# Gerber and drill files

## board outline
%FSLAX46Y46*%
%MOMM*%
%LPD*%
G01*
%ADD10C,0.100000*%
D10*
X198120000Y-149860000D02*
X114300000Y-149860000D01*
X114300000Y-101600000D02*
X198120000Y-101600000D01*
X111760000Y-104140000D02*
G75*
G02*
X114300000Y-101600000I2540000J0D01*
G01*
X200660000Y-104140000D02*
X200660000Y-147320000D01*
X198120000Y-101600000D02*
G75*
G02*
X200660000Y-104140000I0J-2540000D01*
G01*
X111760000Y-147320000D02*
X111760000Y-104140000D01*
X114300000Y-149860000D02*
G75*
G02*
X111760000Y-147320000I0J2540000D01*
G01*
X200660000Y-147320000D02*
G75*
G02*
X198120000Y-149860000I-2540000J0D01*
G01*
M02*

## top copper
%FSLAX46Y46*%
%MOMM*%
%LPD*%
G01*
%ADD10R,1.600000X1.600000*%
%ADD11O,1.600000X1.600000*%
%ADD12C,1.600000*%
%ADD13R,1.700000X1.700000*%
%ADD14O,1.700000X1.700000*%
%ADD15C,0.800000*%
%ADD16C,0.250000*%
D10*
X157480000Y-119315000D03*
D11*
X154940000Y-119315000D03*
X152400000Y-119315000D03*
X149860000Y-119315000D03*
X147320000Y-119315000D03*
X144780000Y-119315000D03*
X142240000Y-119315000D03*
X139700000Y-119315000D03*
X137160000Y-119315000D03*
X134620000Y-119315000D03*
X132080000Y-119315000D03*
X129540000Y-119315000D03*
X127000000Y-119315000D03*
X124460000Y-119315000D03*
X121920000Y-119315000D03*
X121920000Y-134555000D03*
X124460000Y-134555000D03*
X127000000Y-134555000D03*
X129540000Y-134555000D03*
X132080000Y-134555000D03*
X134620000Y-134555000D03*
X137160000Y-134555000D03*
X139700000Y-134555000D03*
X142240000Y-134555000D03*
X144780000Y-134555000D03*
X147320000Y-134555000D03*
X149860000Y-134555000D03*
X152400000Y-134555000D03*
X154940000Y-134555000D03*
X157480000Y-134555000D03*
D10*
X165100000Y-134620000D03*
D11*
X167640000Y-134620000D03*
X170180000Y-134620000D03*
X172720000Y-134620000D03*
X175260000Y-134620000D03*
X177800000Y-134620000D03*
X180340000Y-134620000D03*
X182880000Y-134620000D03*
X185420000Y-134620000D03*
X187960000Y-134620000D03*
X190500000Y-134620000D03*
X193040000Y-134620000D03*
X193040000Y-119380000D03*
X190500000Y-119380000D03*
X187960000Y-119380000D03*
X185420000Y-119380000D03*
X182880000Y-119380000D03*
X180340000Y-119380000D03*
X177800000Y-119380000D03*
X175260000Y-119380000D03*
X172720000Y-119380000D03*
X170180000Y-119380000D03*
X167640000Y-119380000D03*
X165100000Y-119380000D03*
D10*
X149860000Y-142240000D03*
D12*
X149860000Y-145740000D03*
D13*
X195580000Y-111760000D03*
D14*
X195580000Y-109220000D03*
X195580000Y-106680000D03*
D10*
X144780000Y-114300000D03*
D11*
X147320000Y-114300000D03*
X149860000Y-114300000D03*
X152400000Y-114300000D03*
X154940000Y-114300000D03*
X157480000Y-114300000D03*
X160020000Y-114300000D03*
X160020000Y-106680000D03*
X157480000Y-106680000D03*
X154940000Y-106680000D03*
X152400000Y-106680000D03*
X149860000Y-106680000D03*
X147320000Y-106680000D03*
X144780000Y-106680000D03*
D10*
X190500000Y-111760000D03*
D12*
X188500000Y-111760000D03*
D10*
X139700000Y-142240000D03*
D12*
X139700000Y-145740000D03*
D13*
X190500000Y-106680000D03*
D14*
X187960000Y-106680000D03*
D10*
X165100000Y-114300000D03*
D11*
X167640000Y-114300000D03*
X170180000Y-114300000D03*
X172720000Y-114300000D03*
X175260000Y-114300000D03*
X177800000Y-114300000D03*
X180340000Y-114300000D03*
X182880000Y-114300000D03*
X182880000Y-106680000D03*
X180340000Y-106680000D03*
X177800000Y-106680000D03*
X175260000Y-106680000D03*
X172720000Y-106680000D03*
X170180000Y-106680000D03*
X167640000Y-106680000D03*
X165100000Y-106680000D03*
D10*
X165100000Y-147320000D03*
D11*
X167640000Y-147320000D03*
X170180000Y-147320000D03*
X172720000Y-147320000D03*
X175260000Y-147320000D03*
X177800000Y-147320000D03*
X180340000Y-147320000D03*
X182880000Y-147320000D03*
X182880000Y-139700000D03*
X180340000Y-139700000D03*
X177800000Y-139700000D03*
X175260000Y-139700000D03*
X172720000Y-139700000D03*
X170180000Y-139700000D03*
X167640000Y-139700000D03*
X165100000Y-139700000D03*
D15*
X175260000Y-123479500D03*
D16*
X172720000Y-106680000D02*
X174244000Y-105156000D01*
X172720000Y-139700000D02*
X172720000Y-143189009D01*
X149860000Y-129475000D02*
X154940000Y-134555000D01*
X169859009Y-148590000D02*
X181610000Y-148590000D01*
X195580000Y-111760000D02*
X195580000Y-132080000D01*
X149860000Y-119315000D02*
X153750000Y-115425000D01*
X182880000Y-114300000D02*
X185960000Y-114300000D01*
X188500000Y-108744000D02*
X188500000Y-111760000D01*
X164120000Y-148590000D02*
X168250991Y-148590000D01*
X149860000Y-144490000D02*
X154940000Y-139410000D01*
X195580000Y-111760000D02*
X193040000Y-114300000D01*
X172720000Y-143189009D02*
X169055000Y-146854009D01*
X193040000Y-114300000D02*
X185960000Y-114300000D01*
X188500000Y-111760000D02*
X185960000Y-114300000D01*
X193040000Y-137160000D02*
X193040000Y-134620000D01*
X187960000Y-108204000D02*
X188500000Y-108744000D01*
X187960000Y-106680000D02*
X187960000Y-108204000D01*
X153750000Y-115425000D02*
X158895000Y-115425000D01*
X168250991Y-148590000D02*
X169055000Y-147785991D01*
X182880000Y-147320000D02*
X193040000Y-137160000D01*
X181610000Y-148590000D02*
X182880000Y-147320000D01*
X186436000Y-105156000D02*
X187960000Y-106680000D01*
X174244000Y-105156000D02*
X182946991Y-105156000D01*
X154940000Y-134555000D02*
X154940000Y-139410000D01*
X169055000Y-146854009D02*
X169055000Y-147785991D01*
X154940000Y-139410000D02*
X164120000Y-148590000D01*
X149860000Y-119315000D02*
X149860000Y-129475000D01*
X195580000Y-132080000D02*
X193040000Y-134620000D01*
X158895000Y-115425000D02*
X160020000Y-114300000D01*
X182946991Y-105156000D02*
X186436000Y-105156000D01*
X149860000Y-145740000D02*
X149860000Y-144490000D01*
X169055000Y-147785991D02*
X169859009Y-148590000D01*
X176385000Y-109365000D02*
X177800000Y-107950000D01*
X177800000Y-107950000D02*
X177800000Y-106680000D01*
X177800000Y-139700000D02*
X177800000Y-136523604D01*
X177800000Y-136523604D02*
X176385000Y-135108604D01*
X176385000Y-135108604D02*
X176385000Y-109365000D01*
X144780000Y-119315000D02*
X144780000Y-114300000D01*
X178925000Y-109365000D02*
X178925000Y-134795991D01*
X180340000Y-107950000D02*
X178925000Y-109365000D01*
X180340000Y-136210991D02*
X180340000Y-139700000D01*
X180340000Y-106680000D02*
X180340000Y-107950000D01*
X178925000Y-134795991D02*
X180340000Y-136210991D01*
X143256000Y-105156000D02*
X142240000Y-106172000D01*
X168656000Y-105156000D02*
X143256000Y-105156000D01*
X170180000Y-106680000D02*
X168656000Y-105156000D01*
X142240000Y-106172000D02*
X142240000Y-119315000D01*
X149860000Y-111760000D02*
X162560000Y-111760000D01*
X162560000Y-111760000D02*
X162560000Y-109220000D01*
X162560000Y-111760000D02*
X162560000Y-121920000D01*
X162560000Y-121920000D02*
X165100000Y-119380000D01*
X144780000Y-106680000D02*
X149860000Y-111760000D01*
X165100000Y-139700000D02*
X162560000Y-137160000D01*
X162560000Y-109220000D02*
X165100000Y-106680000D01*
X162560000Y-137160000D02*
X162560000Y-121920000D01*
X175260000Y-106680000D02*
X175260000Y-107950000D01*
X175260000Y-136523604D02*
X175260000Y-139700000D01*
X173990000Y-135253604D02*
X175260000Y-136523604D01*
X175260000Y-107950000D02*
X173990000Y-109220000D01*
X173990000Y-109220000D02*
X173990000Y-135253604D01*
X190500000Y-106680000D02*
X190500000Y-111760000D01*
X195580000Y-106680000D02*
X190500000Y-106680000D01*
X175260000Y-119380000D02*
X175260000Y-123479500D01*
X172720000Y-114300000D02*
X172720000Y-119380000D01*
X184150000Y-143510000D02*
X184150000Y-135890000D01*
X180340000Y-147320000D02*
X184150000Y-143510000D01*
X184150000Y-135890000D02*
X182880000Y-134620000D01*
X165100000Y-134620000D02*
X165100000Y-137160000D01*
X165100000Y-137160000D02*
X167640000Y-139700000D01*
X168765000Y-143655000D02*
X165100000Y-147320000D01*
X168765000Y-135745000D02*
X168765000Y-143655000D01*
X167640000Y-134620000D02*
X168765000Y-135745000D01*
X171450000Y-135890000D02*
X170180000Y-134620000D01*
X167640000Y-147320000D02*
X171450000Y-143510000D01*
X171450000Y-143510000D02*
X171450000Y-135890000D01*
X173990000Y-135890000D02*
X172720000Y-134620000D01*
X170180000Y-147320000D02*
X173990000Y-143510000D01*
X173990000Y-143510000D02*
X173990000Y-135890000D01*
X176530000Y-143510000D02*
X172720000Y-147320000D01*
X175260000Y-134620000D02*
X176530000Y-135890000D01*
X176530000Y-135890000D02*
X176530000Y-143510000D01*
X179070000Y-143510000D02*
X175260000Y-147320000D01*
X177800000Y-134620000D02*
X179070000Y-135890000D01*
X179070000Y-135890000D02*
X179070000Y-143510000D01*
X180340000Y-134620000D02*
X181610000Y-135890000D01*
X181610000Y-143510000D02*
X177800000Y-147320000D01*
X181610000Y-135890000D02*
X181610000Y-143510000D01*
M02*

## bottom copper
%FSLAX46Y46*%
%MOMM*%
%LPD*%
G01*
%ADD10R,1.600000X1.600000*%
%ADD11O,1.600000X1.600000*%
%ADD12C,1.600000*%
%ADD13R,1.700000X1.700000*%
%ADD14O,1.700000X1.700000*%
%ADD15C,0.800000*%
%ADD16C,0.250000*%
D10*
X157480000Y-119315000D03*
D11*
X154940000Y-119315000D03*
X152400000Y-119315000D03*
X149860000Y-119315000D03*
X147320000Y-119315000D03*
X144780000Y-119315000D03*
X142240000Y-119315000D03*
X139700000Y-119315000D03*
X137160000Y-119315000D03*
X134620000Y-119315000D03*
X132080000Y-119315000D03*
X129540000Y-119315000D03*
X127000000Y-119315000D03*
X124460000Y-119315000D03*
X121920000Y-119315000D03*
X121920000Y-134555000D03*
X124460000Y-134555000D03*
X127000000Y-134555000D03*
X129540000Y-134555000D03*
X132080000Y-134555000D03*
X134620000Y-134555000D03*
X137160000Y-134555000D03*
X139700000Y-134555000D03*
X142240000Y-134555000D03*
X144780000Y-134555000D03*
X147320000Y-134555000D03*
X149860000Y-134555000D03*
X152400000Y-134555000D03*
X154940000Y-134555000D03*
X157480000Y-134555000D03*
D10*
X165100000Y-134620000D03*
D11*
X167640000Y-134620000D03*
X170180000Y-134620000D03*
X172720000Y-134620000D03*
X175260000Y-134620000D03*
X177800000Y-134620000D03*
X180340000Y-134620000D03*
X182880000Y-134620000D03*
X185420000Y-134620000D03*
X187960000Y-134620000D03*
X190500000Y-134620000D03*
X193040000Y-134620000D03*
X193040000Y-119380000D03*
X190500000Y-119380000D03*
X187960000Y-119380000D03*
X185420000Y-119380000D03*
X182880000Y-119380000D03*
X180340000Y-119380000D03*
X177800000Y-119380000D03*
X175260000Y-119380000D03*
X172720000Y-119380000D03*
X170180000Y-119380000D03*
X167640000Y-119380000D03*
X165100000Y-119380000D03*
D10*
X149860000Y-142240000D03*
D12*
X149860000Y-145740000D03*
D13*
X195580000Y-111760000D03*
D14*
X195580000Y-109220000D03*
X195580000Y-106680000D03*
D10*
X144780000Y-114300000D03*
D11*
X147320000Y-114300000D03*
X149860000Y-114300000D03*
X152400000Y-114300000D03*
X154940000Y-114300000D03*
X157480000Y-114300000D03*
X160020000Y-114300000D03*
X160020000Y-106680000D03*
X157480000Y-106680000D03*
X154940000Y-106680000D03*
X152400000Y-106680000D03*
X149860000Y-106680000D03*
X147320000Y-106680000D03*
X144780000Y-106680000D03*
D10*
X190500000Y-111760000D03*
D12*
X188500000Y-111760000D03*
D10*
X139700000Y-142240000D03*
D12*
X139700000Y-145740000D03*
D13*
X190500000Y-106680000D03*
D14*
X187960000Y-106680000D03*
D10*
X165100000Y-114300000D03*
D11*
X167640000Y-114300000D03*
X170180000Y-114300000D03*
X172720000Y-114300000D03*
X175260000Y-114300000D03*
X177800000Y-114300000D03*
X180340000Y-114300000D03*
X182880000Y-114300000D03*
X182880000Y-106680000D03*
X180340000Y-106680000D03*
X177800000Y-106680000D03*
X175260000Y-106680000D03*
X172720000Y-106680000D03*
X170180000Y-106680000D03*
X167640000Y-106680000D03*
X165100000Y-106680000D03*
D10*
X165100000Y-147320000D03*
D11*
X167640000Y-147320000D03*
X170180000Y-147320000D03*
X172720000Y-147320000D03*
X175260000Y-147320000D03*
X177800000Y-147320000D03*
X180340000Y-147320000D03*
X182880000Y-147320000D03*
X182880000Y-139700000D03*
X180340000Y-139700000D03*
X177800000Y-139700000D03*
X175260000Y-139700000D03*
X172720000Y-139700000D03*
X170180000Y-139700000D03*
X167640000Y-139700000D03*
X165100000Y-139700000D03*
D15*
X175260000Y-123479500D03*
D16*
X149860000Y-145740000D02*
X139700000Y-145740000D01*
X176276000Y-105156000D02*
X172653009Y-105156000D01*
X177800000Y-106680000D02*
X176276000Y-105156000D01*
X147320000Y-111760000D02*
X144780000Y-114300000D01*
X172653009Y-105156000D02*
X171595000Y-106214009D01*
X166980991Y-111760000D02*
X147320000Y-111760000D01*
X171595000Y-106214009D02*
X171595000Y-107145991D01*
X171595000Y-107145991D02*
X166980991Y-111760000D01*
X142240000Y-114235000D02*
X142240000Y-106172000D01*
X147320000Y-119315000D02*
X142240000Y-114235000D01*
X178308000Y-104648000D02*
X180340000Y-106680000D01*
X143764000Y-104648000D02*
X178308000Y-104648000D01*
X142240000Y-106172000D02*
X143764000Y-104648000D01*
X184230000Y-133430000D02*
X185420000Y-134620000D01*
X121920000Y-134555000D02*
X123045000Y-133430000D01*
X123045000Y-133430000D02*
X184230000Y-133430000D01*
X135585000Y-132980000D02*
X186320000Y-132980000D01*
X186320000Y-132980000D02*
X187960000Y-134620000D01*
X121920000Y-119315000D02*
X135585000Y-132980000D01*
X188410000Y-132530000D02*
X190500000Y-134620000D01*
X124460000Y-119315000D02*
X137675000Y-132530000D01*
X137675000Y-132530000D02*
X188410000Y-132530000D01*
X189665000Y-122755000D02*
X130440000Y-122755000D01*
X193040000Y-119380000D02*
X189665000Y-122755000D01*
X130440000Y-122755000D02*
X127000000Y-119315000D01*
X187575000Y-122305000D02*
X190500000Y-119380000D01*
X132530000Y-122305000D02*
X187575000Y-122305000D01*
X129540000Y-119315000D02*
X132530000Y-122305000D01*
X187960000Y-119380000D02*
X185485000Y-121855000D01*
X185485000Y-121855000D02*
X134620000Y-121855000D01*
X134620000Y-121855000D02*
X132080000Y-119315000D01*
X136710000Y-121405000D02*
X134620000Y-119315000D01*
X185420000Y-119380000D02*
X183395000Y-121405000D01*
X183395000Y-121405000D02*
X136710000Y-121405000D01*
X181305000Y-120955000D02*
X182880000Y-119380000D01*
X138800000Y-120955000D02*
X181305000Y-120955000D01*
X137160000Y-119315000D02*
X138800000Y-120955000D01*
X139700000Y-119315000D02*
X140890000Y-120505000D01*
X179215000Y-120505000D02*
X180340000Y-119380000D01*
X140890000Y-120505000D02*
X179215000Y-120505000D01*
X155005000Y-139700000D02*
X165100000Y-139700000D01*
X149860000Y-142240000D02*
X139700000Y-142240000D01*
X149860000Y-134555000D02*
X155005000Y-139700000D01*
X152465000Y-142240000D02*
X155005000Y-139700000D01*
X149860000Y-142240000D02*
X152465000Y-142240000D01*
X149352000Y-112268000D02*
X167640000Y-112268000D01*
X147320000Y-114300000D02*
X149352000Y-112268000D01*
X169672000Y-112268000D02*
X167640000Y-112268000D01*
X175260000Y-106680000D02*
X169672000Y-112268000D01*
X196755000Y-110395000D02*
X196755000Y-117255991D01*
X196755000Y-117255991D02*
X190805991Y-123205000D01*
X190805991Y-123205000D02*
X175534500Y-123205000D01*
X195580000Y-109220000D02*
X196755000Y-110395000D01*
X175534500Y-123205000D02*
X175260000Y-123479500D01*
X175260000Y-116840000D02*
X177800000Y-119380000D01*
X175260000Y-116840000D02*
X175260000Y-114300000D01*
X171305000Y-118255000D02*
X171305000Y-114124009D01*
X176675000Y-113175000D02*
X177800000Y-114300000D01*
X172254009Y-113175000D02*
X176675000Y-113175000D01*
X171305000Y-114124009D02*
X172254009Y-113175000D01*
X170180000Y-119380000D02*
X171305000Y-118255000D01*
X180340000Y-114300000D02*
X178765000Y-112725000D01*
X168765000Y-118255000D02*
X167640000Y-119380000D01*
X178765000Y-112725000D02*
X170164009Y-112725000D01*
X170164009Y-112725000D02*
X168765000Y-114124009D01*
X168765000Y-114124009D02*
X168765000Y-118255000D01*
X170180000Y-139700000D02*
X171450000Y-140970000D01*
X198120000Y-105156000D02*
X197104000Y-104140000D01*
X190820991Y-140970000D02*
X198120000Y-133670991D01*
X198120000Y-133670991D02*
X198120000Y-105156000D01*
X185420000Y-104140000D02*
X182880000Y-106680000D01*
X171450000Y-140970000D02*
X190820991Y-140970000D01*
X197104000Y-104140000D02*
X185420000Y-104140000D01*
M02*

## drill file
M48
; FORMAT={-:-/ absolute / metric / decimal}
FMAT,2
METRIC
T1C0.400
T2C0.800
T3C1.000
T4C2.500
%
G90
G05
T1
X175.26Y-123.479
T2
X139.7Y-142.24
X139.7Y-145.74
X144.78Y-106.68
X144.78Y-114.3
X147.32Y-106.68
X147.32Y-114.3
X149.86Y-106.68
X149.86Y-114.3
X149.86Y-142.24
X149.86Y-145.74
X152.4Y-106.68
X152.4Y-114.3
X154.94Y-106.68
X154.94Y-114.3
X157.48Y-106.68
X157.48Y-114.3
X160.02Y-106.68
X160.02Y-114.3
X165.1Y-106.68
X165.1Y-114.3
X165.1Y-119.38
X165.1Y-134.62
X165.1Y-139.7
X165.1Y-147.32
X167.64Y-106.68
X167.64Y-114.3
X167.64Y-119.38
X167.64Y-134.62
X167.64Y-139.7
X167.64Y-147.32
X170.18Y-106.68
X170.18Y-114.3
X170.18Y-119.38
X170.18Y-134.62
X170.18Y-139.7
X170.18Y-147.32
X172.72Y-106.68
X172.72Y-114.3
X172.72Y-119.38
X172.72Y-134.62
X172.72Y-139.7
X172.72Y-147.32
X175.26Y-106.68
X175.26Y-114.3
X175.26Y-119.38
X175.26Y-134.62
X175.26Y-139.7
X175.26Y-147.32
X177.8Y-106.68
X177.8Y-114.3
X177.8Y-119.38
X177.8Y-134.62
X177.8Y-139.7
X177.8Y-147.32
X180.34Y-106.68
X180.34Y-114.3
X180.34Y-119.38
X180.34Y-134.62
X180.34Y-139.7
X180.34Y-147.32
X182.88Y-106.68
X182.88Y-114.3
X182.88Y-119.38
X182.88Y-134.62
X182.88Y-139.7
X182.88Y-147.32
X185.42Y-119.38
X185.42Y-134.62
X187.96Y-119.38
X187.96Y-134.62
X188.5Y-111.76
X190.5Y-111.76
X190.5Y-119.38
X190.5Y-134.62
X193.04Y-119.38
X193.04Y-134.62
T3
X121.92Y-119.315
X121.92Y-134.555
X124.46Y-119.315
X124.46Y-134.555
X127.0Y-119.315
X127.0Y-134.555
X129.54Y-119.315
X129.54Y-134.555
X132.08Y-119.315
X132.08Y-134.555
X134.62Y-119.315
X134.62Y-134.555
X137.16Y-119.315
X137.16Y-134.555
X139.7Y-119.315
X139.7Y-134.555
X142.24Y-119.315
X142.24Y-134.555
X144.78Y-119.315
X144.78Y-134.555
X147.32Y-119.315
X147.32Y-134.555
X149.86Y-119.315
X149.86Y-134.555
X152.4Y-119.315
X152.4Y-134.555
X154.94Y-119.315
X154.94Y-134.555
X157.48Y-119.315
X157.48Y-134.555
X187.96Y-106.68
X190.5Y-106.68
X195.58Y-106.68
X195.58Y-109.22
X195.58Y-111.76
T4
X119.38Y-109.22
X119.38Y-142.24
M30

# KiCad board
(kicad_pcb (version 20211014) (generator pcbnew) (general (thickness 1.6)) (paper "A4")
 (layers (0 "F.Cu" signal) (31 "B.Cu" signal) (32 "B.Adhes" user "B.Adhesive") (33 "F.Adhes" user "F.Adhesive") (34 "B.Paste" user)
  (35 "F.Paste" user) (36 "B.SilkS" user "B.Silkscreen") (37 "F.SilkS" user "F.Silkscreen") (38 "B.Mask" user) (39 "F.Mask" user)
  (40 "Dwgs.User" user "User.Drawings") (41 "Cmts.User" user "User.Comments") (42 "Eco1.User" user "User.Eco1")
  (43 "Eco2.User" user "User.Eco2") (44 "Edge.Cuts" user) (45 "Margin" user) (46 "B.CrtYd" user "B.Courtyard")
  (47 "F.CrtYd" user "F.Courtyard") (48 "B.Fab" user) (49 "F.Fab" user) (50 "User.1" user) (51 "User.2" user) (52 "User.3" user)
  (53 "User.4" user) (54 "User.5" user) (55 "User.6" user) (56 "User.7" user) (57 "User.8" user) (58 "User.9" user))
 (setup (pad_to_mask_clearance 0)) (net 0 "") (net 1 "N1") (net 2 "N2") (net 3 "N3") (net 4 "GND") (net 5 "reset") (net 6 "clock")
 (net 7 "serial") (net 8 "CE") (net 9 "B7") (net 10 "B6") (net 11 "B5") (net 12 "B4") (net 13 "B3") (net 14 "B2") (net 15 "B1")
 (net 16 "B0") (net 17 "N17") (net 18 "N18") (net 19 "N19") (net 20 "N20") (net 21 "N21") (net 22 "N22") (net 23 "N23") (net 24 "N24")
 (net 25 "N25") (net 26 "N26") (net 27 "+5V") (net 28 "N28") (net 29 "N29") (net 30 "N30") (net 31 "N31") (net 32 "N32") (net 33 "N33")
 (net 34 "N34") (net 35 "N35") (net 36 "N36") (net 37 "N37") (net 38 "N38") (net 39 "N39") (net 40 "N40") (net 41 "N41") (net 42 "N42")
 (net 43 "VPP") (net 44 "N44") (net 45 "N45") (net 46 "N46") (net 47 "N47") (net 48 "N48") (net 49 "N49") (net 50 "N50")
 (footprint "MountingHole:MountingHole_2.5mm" (layer "F.Cu") (at 119.38 109.22)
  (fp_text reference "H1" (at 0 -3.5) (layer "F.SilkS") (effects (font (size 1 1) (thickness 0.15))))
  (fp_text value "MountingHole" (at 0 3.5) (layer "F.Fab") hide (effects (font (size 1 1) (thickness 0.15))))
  (pad "" np_thru_hole circle (at 0 0) (size 2.5 2.5) (drill 2.5) (layers *.Cu *.Mask)))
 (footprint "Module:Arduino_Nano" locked (layer "F.Cu") (at 157.48 119.315 -90)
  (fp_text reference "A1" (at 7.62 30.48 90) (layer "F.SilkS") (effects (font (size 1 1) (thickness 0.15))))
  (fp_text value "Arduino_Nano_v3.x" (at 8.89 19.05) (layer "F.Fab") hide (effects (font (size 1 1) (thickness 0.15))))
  (pad "1" thru_hole rect locked (at 0 0 270) (size 1.6 1.6) (drill 1) (layers *.Cu *.Mask) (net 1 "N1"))
  (pad "2" thru_hole oval locked (at 0 2.54 270) (size 1.6 1.6) (drill 1) (layers *.Cu *.Mask) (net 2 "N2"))
  (pad "3" thru_hole oval locked (at 0 5.08 270) (size 1.6 1.6) (drill 1) (layers *.Cu *.Mask) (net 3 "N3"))
  (pad "4" thru_hole oval locked (at 0 7.62 270) (size 1.6 1.6) (drill 1) (layers *.Cu *.Mask) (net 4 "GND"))
  (pad "5" thru_hole oval locked (at 0 10.16 270) (size 1.6 1.6) (drill 1) (layers *.Cu *.Mask) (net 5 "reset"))
  (pad "6" thru_hole oval locked (at 0 12.7 270) (size 1.6 1.6) (drill 1) (layers *.Cu *.Mask) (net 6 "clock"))
  (pad "7" thru_hole oval locked (at 0 15.24 270) (size 1.6 1.6) (drill 1) (layers *.Cu *.Mask) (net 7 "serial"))
  (pad "8" thru_hole oval locked (at 0 17.78 270) (size 1.6 1.6) (drill 1) (layers *.Cu *.Mask) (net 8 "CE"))
  (pad "9" thru_hole oval locked (at 0 20.32 270) (size 1.6 1.6) (drill 1) (layers *.Cu *.Mask) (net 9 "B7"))
  (pad "10" thru_hole oval locked (at 0 22.86 270) (size 1.6 1.6) (drill 1) (layers *.Cu *.Mask) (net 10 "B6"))
  (pad "11" thru_hole oval locked (at 0 25.4 270) (size 1.6 1.6) (drill 1) (layers *.Cu *.Mask) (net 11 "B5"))
  (pad "12" thru_hole oval locked (at 0 27.94 270) (size 1.6 1.6) (drill 1) (layers *.Cu *.Mask) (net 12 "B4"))
  (pad "13" thru_hole oval locked (at 0 30.48 270) (size 1.6 1.6) (drill 1) (layers *.Cu *.Mask) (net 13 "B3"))
  (pad "14" thru_hole oval locked (at 0 33.02 270) (size 1.6 1.6) (drill 1) (layers *.Cu *.Mask) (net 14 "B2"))
  (pad "15" thru_hole oval locked (at 0 35.56 270) (size 1.6 1.6) (drill 1) (layers *.Cu *.Mask) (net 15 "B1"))
  (pad "16" thru_hole oval locked (at 15.24 35.56 270) (size 1.6 1.6) (drill 1) (layers *.Cu *.Mask) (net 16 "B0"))
  (pad "17" thru_hole oval locked (at 15.24 33.02 270) (size 1.6 1.6) (drill 1) (layers *.Cu *.Mask) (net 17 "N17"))
  (pad "18" thru_hole oval locked (at 15.24 30.48 270) (size 1.6 1.6) (drill 1) (layers *.Cu *.Mask) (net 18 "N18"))
  (pad "19" thru_hole oval locked (at 15.24 27.94 270) (size 1.6 1.6) (drill 1) (layers *.Cu *.Mask) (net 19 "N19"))
  (pad "20" thru_hole oval locked (at 15.24 25.4 270) (size 1.6 1.6) (drill 1) (layers *.Cu *.Mask) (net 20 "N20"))
  (pad "21" thru_hole oval locked (at 15.24 22.86 270) (size 1.6 1.6) (drill 1) (layers *.Cu *.Mask) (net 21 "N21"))
  (pad "22" thru_hole oval locked (at 15.24 20.32 270) (size 1.6 1.6) (drill 1) (layers *.Cu *.Mask) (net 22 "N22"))
  (pad "23" thru_hole oval locked (at 15.24 17.78 270) (size 1.6 1.6) (drill 1) (layers *.Cu *.Mask) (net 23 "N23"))
  (pad "24" thru_hole oval locked (at 15.24 15.24 270) (size 1.6 1.6) (drill 1) (layers *.Cu *.Mask) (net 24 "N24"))
  (pad "25" thru_hole oval locked (at 15.24 12.7 270) (size 1.6 1.6) (drill 1) (layers *.Cu *.Mask) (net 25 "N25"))
  (pad "26" thru_hole oval locked (at 15.24 10.16 270) (size 1.6 1.6) (drill 1) (layers *.Cu *.Mask) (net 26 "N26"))
  (pad "27" thru_hole oval locked (at 15.24 7.62 270) (size 1.6 1.6) (drill 1) (layers *.Cu *.Mask) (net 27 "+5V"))
  (pad "28" thru_hole oval locked (at 15.24 5.08 270) (size 1.6 1.6) (drill 1) (layers *.Cu *.Mask) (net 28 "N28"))
  (pad "29" thru_hole oval locked (at 15.24 2.54 270) (size 1.6 1.6) (drill 1) (layers *.Cu *.Mask) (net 4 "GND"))
  (pad "30" thru_hole oval locked (at 15.24 0 270) (size 1.6 1.6) (drill 1) (layers *.Cu *.Mask) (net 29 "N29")))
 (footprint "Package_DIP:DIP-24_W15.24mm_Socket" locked (layer "F.Cu") (at 165.1 134.62 90)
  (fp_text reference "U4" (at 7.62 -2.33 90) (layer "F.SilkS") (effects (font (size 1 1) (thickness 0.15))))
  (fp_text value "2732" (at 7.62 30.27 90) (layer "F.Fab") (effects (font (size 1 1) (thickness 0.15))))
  (pad "1" thru_hole rect locked (at 0 0 90) (size 1.6 1.6) (drill 0.8) (layers *.Cu *.Mask) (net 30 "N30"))
  (pad "2" thru_hole oval locked (at 0 2.54 90) (size 1.6 1.6) (drill 0.8) (layers *.Cu *.Mask) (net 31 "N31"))
  (pad "3" thru_hole oval locked (at 0 5.08 90) (size 1.6 1.6) (drill 0.8) (layers *.Cu *.Mask) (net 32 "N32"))
  (pad "4" thru_hole oval locked (at 0 7.62 90) (size 1.6 1.6) (drill 0.8) (layers *.Cu *.Mask) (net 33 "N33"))
  (pad "5" thru_hole oval locked (at 0 10.16 90) (size 1.6 1.6) (drill 0.8) (layers *.Cu *.Mask) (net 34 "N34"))
  (pad "6" thru_hole oval locked (at 0 12.7 90) (size 1.6 1.6) (drill 0.8) (layers *.Cu *.Mask) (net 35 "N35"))
  (pad "7" thru_hole oval locked (at 0 15.24 90) (size 1.6 1.6) (drill 0.8) (layers *.Cu *.Mask) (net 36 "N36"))
  (pad "8" thru_hole oval locked (at 0 17.78 90) (size 1.6 1.6) (drill 0.8) (layers *.Cu *.Mask) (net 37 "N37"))
  (pad "9" thru_hole oval locked (at 0 20.32 90) (size 1.6 1.6) (drill 0.8) (layers *.Cu *.Mask) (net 16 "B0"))
  (pad "10" thru_hole oval locked (at 0 22.86 90) (size 1.6 1.6) (drill 0.8) (layers *.Cu *.Mask) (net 15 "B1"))
  (pad "11" thru_hole oval locked (at 0 25.4 90) (size 1.6 1.6) (drill 0.8) (layers *.Cu *.Mask) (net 14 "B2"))
  (pad "12" thru_hole oval locked (at 0 27.94 90) (size 1.6 1.6) (drill 0.8) (layers *.Cu *.Mask) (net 4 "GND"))
  (pad "13" thru_hole oval locked (at 15.24 27.94 90) (size 1.6 1.6) (drill 0.8) (layers *.Cu *.Mask) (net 13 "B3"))
  (pad "14" thru_hole oval locked (at 15.24 25.4 90) (size 1.6 1.6) (drill 0.8) (layers *.Cu *.Mask) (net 12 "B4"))
  (pad "15" thru_hole oval locked (at 15.24 22.86 90) (size 1.6 1.6) (drill 0.8) (layers *.Cu *.Mask) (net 11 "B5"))
  (pad "16" thru_hole oval locked (at 15.24 20.32 90) (size 1.6 1.6) (drill 0.8) (layers *.Cu *.Mask) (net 10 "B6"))
  (pad "17" thru_hole oval locked (at 15.24 17.78 90) (size 1.6 1.6) (drill 0.8) (layers *.Cu *.Mask) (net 9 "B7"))
  (pad "18" thru_hole oval locked (at 15.24 15.24 90) (size 1.6 1.6) (drill 0.8) (layers *.Cu *.Mask) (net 8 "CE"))
  (pad "19" thru_hole oval locked (at 15.24 12.7 90) (size 1.6 1.6) (drill 0.8) (layers *.Cu *.Mask) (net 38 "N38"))
  (pad "20" thru_hole oval locked (at 15.24 10.16 90) (size 1.6 1.6) (drill 0.8) (layers *.Cu *.Mask) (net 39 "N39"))
  (pad "21" thru_hole oval locked (at 15.24 7.62 90) (size 1.6 1.6) (drill 0.8) (layers *.Cu *.Mask) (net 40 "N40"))
  (pad "22" thru_hole oval locked (at 15.24 5.08 90) (size 1.6 1.6) (drill 0.8) (layers *.Cu *.Mask) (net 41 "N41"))
  (pad "23" thru_hole oval locked (at 15.24 2.54 90) (size 1.6 1.6) (drill 0.8) (layers *.Cu *.Mask) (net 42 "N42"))
  (pad "24" thru_hole oval locked (at 15.24 0 90) (size 1.6 1.6) (drill 0.8) (layers *.Cu *.Mask) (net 27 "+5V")))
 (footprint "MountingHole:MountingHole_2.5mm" (layer "F.Cu") (at 119.38 142.24)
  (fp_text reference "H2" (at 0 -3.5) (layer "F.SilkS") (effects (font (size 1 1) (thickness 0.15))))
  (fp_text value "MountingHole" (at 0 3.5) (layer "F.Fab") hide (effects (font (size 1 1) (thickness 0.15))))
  (pad "" np_thru_hole circle (at 0 0) (size 2.5 2.5) (drill 2.5) (layers *.Cu *.Mask)))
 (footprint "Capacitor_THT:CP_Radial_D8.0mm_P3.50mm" (layer "F.Cu") (at 149.86 142.24 -90)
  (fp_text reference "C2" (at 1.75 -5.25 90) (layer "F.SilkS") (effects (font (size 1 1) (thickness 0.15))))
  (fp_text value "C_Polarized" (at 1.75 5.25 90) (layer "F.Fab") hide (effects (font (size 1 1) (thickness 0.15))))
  (pad "1" thru_hole rect (at 0 0 270) (size 1.6 1.6) (drill 0.8) (layers *.Cu *.Mask) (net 27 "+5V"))
  (pad "2" thru_hole circle (at 3.5 0 270) (size 1.6 1.6) (drill 0.8) (layers *.Cu *.Mask) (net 4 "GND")))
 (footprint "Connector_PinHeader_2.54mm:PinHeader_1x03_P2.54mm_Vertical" (layer "F.Cu") (at 195.58 111.76 180)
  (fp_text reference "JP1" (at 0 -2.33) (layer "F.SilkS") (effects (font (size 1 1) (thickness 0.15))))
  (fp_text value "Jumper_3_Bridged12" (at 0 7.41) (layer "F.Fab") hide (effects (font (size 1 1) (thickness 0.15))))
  (pad "1" thru_hole rect (at 0 0 180) (size 1.7 1.7) (drill 1) (layers *.Cu *.Mask) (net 4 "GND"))
  (pad "2" thru_hole oval (at 0 2.54 180) (size 1.7 1.7) (drill 1) (layers *.Cu *.Mask) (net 39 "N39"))
  (pad "3" thru_hole oval (at 0 5.08 180) (size 1.7 1.7) (drill 1) (layers *.Cu *.Mask) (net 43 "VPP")))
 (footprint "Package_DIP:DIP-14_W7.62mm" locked (layer "F.Cu") (at 144.78 114.3 90)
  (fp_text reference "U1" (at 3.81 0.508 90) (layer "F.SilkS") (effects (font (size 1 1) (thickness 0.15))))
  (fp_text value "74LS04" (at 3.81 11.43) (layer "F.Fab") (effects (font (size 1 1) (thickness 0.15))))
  (pad "1" thru_hole rect locked (at 0 0 90) (size 1.6 1.6) (drill 0.8) (layers *.Cu *.Mask) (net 6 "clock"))
  (pad "2" thru_hole oval locked (at 0 2.54 90) (size 1.6 1.6) (drill 0.8) (layers *.Cu *.Mask) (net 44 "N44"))
  (pad "3" thru_hole oval locked (at 0 5.08 90) (size 1.6 1.6) (drill 0.8) (layers *.Cu *.Mask))
  (pad "4" thru_hole oval locked (at 0 7.62 90) (size 1.6 1.6) (drill 0.8) (layers *.Cu *.Mask))
  (pad "5" thru_hole oval locked (at 0 10.16 90) (size 1.6 1.6) (drill 0.8) (layers *.Cu *.Mask))
  (pad "6" thru_hole oval locked (at 0 12.7 90) (size 1.6 1.6) (drill 0.8) (layers *.Cu *.Mask))
  (pad "7" thru_hole oval locked (at 0 15.24 90) (size 1.6 1.6) (drill 0.8) (layers *.Cu *.Mask) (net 4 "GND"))
  (pad "8" thru_hole oval locked (at 7.62 15.24 90) (size 1.6 1.6) (drill 0.8) (layers *.Cu *.Mask))
  (pad "9" thru_hole oval locked (at 7.62 12.7 90) (size 1.6 1.6) (drill 0.8) (layers *.Cu *.Mask))
  (pad "10" thru_hole oval locked (at 7.62 10.16 90) (size 1.6 1.6) (drill 0.8) (layers *.Cu *.Mask))
  (pad "11" thru_hole oval locked (at 7.62 7.62 90) (size 1.6 1.6) (drill 0.8) (layers *.Cu *.Mask))
  (pad "12" thru_hole oval locked (at 7.62 5.08 90) (size 1.6 1.6) (drill 0.8) (layers *.Cu *.Mask))
  (pad "13" thru_hole oval locked (at 7.62 2.54 90) (size 1.6 1.6) (drill 0.8) (layers *.Cu *.Mask))
  (pad "14" thru_hole oval locked (at 7.62 0 90) (size 1.6 1.6) (drill 0.8) (layers *.Cu *.Mask) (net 27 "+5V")))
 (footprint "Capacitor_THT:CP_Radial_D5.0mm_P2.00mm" (layer "F.Cu") (at 190.5 111.76 180)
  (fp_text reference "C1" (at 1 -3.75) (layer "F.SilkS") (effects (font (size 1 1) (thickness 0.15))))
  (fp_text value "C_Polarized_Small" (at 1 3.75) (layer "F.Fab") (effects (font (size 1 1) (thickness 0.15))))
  (pad "1" thru_hole rect (at 0 0 180) (size 1.6 1.6) (drill 0.8) (layers *.Cu *.Mask) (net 43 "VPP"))
  (pad "2" thru_hole circle (at 2 0 180) (size 1.6 1.6) (drill 0.8) (layers *.Cu *.Mask) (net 4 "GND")))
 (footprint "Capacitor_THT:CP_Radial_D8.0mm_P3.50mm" (layer "F.Cu") (at 139.7 142.24 -90)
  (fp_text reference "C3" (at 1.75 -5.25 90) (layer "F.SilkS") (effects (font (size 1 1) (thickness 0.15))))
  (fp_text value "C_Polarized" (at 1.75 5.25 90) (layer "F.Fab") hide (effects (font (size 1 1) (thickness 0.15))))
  (pad "1" thru_hole rect (at 0 0 270) (size 1.6 1.6) (drill 0.8) (layers *.Cu *.Mask) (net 27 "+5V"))
  (pad "2" thru_hole circle (at 3.5 0 270) (size 1.6 1.6) (drill 0.8) (layers *.Cu *.Mask) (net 4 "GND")))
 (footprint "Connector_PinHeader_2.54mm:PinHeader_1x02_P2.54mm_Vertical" (layer "F.Cu") (at 190.5 106.68 -90)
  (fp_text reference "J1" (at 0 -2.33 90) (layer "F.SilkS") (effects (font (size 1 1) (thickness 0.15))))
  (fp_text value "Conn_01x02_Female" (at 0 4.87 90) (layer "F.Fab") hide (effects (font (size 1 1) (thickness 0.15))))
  (pad "1" thru_hole rect (at 0 0 270) (size 1.7 1.7) (drill 1) (layers *.Cu *.Mask) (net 43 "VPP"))
  (pad "2" thru_hole oval (at 0 2.54 270) (size 1.7 1.7) (drill 1) (layers *.Cu *.Mask) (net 4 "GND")))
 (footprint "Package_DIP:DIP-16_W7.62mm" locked (layer "F.Cu") (at 165.1 114.3 90)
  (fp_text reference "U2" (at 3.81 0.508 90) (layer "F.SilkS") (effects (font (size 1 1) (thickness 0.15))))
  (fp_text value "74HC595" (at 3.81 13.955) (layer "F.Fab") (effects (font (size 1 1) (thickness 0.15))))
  (pad "1" thru_hole rect locked (at 0 0 90) (size 1.6 1.6) (drill 0.8) (layers *.Cu *.Mask) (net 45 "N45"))
  (pad "2" thru_hole oval locked (at 0 2.54 90) (size 1.6 1.6) (drill 0.8) (layers *.Cu *.Mask) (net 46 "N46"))
  (pad "3" thru_hole oval locked (at 0 5.08 90) (size 1.6 1.6) (drill 0.8) (layers *.Cu *.Mask) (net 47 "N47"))
  (pad "4" thru_hole oval locked (at 0 7.62 90) (size 1.6 1.6) (drill 0.8) (layers *.Cu *.Mask) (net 40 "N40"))
  (pad "5" thru_hole oval locked (at 0 10.16 90) (size 1.6 1.6) (drill 0.8) (layers *.Cu *.Mask) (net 38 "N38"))
  (pad "6" thru_hole oval locked (at 0 12.7 90) (size 1.6 1.6) (drill 0.8) (layers *.Cu *.Mask) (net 41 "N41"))
  (pad "7" thru_hole oval locked (at 0 15.24 90) (size 1.6 1.6) (drill 0.8) (layers *.Cu *.Mask) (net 42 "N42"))
  (pad "8" thru_hole oval locked (at 0 17.78 90) (size 1.6 1.6) (drill 0.8) (layers *.Cu *.Mask) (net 4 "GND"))
  (pad "9" thru_hole oval locked (at 7.62 17.78 90) (size 1.6 1.6) (drill 0.8) (layers *.Cu *.Mask) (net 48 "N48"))
  (pad "10" thru_hole oval locked (at 7.62 15.24 90) (size 1.6 1.6) (drill 0.8) (layers *.Cu *.Mask) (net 5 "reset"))
  (pad "11" thru_hole oval locked (at 7.62 12.7 90) (size 1.6 1.6) (drill 0.8) (layers *.Cu *.Mask) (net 6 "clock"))
  (pad "12" thru_hole oval locked (at 7.62 10.16 90) (size 1.6 1.6) (drill 0.8) (layers *.Cu *.Mask) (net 44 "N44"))
  (pad "13" thru_hole oval locked (at 7.62 7.62 90) (size 1.6 1.6) (drill 0.8) (layers *.Cu *.Mask) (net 4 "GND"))
  (pad "14" thru_hole oval locked (at 7.62 5.08 90) (size 1.6 1.6) (drill 0.8) (layers *.Cu *.Mask) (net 7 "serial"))
  (pad "15" thru_hole oval locked (at 7.62 2.54 90) (size 1.6 1.6) (drill 0.8) (layers *.Cu *.Mask) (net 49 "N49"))
  (pad "16" thru_hole oval locked (at 7.62 0 90) (size 1.6 1.6) (drill 0.8) (layers *.Cu *.Mask) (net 27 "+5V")))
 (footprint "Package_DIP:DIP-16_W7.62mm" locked (layer "F.Cu") (at 165.1 147.32 90)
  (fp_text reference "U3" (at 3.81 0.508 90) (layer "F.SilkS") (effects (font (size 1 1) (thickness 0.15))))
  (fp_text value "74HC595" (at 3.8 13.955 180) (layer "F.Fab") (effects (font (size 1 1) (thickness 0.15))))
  (pad "1" thru_hole rect locked (at 0 0 90) (size 1.6 1.6) (drill 0.8) (layers *.Cu *.Mask) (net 31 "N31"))
  (pad "2" thru_hole oval locked (at 0 2.54 90) (size 1.6 1.6) (drill 0.8) (layers *.Cu *.Mask) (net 32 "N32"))
  (pad "3" thru_hole oval locked (at 0 5.08 90) (size 1.6 1.6) (drill 0.8) (layers *.Cu *.Mask) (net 33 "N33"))
  (pad "4" thru_hole oval locked (at 0 7.62 90) (size 1.6 1.6) (drill 0.8) (layers *.Cu *.Mask) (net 34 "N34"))
  (pad "5" thru_hole oval locked (at 0 10.16 90) (size 1.6 1.6) (drill 0.8) (layers *.Cu *.Mask) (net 35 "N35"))
  (pad "6" thru_hole oval locked (at 0 12.7 90) (size 1.6 1.6) (drill 0.8) (layers *.Cu *.Mask) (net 36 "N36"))
  (pad "7" thru_hole oval locked (at 0 15.24 90) (size 1.6 1.6) (drill 0.8) (layers *.Cu *.Mask) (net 37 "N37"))
  (pad "8" thru_hole oval locked (at 0 17.78 90) (size 1.6 1.6) (drill 0.8) (layers *.Cu *.Mask) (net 4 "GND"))
  (pad "9" thru_hole oval locked (at 7.62 17.78 90) (size 1.6 1.6) (drill 0.8) (layers *.Cu *.Mask) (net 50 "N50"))
  (pad "10" thru_hole oval locked (at 7.62 15.24 90) (size 1.6 1.6) (drill 0.8) (layers *.Cu *.Mask) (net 5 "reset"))
  (pad "11" thru_hole oval locked (at 7.62 12.7 90) (size 1.6 1.6) (drill 0.8) (layers *.Cu *.Mask) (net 6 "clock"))
  (pad "12" thru_hole oval locked (at 7.62 10.16 90) (size 1.6 1.6) (drill 0.8) (layers *.Cu *.Mask) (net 44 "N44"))
  (pad "13" thru_hole oval locked (at 7.62 7.62 90) (size 1.6 1.6) (drill 0.8) (layers *.Cu *.Mask) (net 4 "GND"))
  (pad "14" thru_hole oval locked (at 7.62 5.08 90) (size 1.6 1.6) (drill 0.8) (layers *.Cu *.Mask) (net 48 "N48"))
  (pad "15" thru_hole oval locked (at 7.62 2.54 90) (size 1.6 1.6) (drill 0.8) (layers *.Cu *.Mask) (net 30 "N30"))
  (pad "16" thru_hole oval locked (at 7.62 0 90) (size 1.6 1.6) (drill 0.8) (layers *.Cu *.Mask) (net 27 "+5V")))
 (gr_line (start 198.12 149.86) (end 114.3 149.86) (layer "Edge.Cuts") (width 0.1))
 (gr_line (start 114.3 101.6) (end 198.12 101.6) (layer "Edge.Cuts") (width 0.1))
 (gr_arc (start 111.76 104.14) (mid 112.503949 102.343949) (end 114.3 101.6) (layer "Edge.Cuts") (width 0.1))
 (gr_line (start 200.66 104.14) (end 200.66 147.32) (layer "Edge.Cuts") (width 0.1))
 (gr_arc (start 198.12 101.6) (mid 199.916051 102.343949) (end 200.66 104.14) (layer "Edge.Cuts") (width 0.1))
 (gr_line (start 111.76 147.32) (end 111.76 104.14) (layer "Edge.Cuts") (width 0.1))
 (gr_arc (start 114.3 149.86) (mid 112.503949 149.116051) (end 111.76 147.32) (layer "Edge.Cuts") (width 0.1))
 (gr_arc (start 200.66 147.32) (mid 199.916051 149.116051) (end 198.12 149.86) (layer "Edge.Cuts") (width 0.1))
 (segment (start 172.72 106.68) (end 174.244 105.156) (width 0.25) (layer "F.Cu") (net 4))
 (segment (start 172.72 139.7) (end 172.72 143.189009) (width 0.25) (layer "F.Cu") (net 4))
 (segment (start 149.86 129.475) (end 154.94 134.555) (width 0.25) (layer "F.Cu") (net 4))
 (segment (start 169.859009 148.59) (end 181.61 148.59) (width 0.25) (layer "F.Cu") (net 4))
 (segment (start 195.58 111.76) (end 195.58 132.08) (width 0.25) (layer "F.Cu") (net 4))
 (segment (start 149.86 119.315) (end 153.75 115.425) (width 0.25) (layer "F.Cu") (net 4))
 (segment (start 182.88 114.3) (end 185.96 114.3) (width 0.25) (layer "F.Cu") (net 4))
 (segment (start 188.5 108.744) (end 188.5 111.76) (width 0.25) (layer "F.Cu") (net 4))
 (segment (start 164.12 148.59) (end 168.250991 148.59) (width 0.25) (layer "F.Cu") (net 4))
 (segment (start 149.86 144.49) (end 154.94 139.41) (width 0.25) (layer "F.Cu") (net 4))
 (segment (start 195.58 111.76) (end 193.04 114.3) (width 0.25) (layer "F.Cu") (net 4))
 (segment (start 172.72 143.189009) (end 169.055 146.854009) (width 0.25) (layer "F.Cu") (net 4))
 (segment (start 193.04 114.3) (end 185.96 114.3) (width 0.25) (layer "F.Cu") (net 4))
 (segment (start 188.5 111.76) (end 185.96 114.3) (width 0.25) (layer "F.Cu") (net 4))
 (segment (start 193.04 137.16) (end 193.04 134.62) (width 0.25) (layer "F.Cu") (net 4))
 (segment (start 187.96 108.204) (end 188.5 108.744) (width 0.25) (layer "F.Cu") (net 4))
 (segment (start 187.96 106.68) (end 187.96 108.204) (width 0.25) (layer "F.Cu") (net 4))
 (segment (start 153.75 115.425) (end 158.895 115.425) (width 0.25) (layer "F.Cu") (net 4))
 (segment (start 168.250991 148.59) (end 169.055 147.785991) (width 0.25) (layer "F.Cu") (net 4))
 (segment (start 182.88 147.32) (end 193.04 137.16) (width 0.25) (layer "F.Cu") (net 4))
 (segment (start 181.61 148.59) (end 182.88 147.32) (width 0.25) (layer "F.Cu") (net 4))
 (segment (start 186.436 105.156) (end 187.96 106.68) (width 0.25) (layer "F.Cu") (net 4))
 (segment (start 174.244 105.156) (end 182.946991 105.156) (width 0.25) (layer "F.Cu") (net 4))
 (segment (start 154.94 134.555) (end 154.94 139.41) (width 0.25) (layer "F.Cu") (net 4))
 (segment (start 169.055 146.854009) (end 169.055 147.785991) (width 0.25) (layer "F.Cu") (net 4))
 (segment (start 154.94 139.41) (end 164.12 148.59) (width 0.25) (layer "F.Cu") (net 4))
 (segment (start 149.86 119.315) (end 149.86 129.475) (width 0.25) (layer "F.Cu") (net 4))
 (segment (start 195.58 132.08) (end 193.04 134.62) (width 0.25) (layer "F.Cu") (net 4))
 (segment (start 158.895 115.425) (end 160.02 114.3) (width 0.25) (layer "F.Cu") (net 4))
 (segment (start 182.946991 105.156) (end 186.436 105.156) (width 0.25) (layer "F.Cu") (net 4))
 (segment (start 149.86 145.74) (end 149.86 144.49) (width 0.25) (layer "F.Cu") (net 4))
 (segment (start 169.055 147.785991) (end 169.859009 148.59) (width 0.25) (layer "F.Cu") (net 4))
 (segment (start 149.86 145.74) (end 139.7 145.74) (width 0.25) (layer "B.Cu") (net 4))
 (segment (start 176.385 109.365) (end 177.8 107.95) (width 0.25) (layer "F.Cu") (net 6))
 (segment (start 177.8 107.95) (end 177.8 106.68) (width 0.25) (layer "F.Cu") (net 6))
 (segment (start 177.8 139.7) (end 177.8 136.523604) (width 0.25) (layer "F.Cu") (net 6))
 (segment (start 177.8 136.523604) (end 176.385 135.108604) (width 0.25) (layer "F.Cu") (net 6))
 (segment (start 176.385 135.108604) (end 176.385 109.365) (width 0.25) (layer "F.Cu") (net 6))
 (segment (start 144.78 119.315) (end 144.78 114.3) (width 0.25) (layer "F.Cu") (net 6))
 (segment (start 176.276 105.156) (end 172.653009 105.156) (width 0.25) (layer "B.Cu") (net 6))
 (segment (start 177.8 106.68) (end 176.276 105.156) (width 0.25) (layer "B.Cu") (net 6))
 (segment (start 147.32 111.76) (end 144.78 114.3) (width 0.25) (layer "B.Cu") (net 6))
 (segment (start 172.653009 105.156) (end 171.595 106.214009) (width 0.25) (layer "B.Cu") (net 6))
 (segment (start 166.980991 111.76) (end 147.32 111.76) (width 0.25) (layer "B.Cu") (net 6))
 (segment (start 171.595 106.214009) (end 171.595 107.145991) (width 0.25) (layer "B.Cu") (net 6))
 (segment (start 171.595 107.145991) (end 166.980991 111.76) (width 0.25) (layer "B.Cu") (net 6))
 (segment (start 178.925 109.365) (end 178.925 134.795991) (width 0.25) (layer "F.Cu") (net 5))
 (segment (start 180.34 107.95) (end 178.925 109.365) (width 0.25) (layer "F.Cu") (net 5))
 (segment (start 180.34 136.210991) (end 180.34 139.7) (width 0.25) (layer "F.Cu") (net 5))
 (segment (start 180.34 106.68) (end 180.34 107.95) (width 0.25) (layer "F.Cu") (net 5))
 (segment (start 178.925 134.795991) (end 180.34 136.210991) (width 0.25) (layer "F.Cu") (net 5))
 (segment (start 142.24 114.235) (end 142.24 106.172) (width 0.25) (layer "B.Cu") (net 5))
 (segment (start 147.32 119.315) (end 142.24 114.235) (width 0.25) (layer "B.Cu") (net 5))
 (segment (start 178.308 104.648) (end 180.34 106.68) (width 0.25) (layer "B.Cu") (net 5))
 (segment (start 143.764 104.648) (end 178.308 104.648) (width 0.25) (layer "B.Cu") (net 5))
 (segment (start 142.24 106.172) (end 143.764 104.648) (width 0.25) (layer "B.Cu") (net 5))
 (segment (start 143.256 105.156) (end 142.24 106.172) (width 0.25) (layer "F.Cu") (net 7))
 (segment (start 168.656 105.156) (end 143.256 105.156) (width 0.25) (layer "F.Cu") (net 7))
 (segment (start 170.18 106.68) (end 168.656 105.156) (width 0.25) (layer "F.Cu") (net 7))
 (segment (start 142.24 106.172) (end 142.24 119.315) (width 0.25) (layer "F.Cu") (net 7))
 (segment (start 184.23 133.43) (end 185.42 134.62) (width 0.25) (layer "B.Cu") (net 16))
 (segment (start 121.92 134.555) (end 123.045 133.43) (width 0.25) (layer "B.Cu") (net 16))
 (segment (start 123.045 133.43) (end 184.23 133.43) (width 0.25) (layer "B.Cu") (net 16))
 (segment (start 135.585 132.98) (end 186.32 132.98) (width 0.25) (layer "B.Cu") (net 15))
 (segment (start 186.32 132.98) (end 187.96 134.62) (width 0.25) (layer "B.Cu") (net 15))
 (segment (start 121.92 119.315) (end 135.585 132.98) (width 0.25) (layer "B.Cu") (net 15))
 (segment (start 188.41 132.53) (end 190.5 134.62) (width 0.25) (layer "B.Cu") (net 14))
 (segment (start 124.46 119.315) (end 137.675 132.53) (width 0.25) (layer "B.Cu") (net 14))
 (segment (start 137.675 132.53) (end 188.41 132.53) (width 0.25) (layer "B.Cu") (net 14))
 (segment (start 189.665 122.755) (end 130.44 122.755) (width 0.25) (layer "B.Cu") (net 13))
 (segment (start 193.04 119.38) (end 189.665 122.755) (width 0.25) (layer "B.Cu") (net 13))
 (segment (start 130.44 122.755) (end 127 119.315) (width 0.25) (layer "B.Cu") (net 13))
 (segment (start 187.575 122.305) (end 190.5 119.38) (width 0.25) (layer "B.Cu") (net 12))
 (segment (start 132.53 122.305) (end 187.575 122.305) (width 0.25) (layer "B.Cu") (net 12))
 (segment (start 129.54 119.315) (end 132.53 122.305) (width 0.25) (layer "B.Cu") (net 12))
 (segment (start 187.96 119.38) (end 185.485 121.855) (width 0.25) (layer "B.Cu") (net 11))
 (segment (start 185.485 121.855) (end 134.62 121.855) (width 0.25) (layer "B.Cu") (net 11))
 (segment (start 134.62 121.855) (end 132.08 119.315) (width 0.25) (layer "B.Cu") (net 11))
 (segment (start 136.71 121.405) (end 134.62 119.315) (width 0.25) (layer "B.Cu") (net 10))
 (segment (start 185.42 119.38) (end 183.395 121.405) (width 0.25) (layer "B.Cu") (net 10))
 (segment (start 183.395 121.405) (end 136.71 121.405) (width 0.25) (layer "B.Cu") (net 10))
 (segment (start 181.305 120.955) (end 182.88 119.38) (width 0.25) (layer "B.Cu") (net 9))
 (segment (start 138.8 120.955) (end 181.305 120.955) (width 0.25) (layer "B.Cu") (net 9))
 (segment (start 137.16 119.315) (end 138.8 120.955) (width 0.25) (layer "B.Cu") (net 9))
 (segment (start 139.7 119.315) (end 140.89 120.505) (width 0.25) (layer "B.Cu") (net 8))
 (segment (start 179.215 120.505) (end 180.34 119.38) (width 0.25) (layer "B.Cu") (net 8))
 (segment (start 140.89 120.505) (end 179.215 120.505) (width 0.25) (layer "B.Cu") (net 8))
 (segment (start 149.86 111.76) (end 162.56 111.76) (width 0.25) (layer "F.Cu") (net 27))
 (segment (start 162.56 111.76) (end 162.56 109.22) (width 0.25) (layer "F.Cu") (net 27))
 (segment (start 162.56 111.76) (end 162.56 121.92) (width 0.25) (layer "F.Cu") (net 27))
 (segment (start 162.56 121.92) (end 165.1 119.38) (width 0.25) (layer "F.Cu") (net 27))
 (segment (start 144.78 106.68) (end 149.86 111.76) (width 0.25) (layer "F.Cu") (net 27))
 (segment (start 165.1 139.7) (end 162.56 137.16) (width 0.25) (layer "F.Cu") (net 27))
 (segment (start 162.56 109.22) (end 165.1 106.68) (width 0.25) (layer "F.Cu") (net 27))
 (segment (start 162.56 137.16) (end 162.56 121.92) (width 0.25) (layer "F.Cu") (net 27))
 (segment (start 155.005 139.7) (end 165.1 139.7) (width 0.25) (layer "B.Cu") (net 27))
 (segment (start 149.86 142.24) (end 139.7 142.24) (width 0.25) (layer "B.Cu") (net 27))
 (segment (start 149.86 134.555) (end 155.005 139.7) (width 0.25) (layer "B.Cu") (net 27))
 (segment (start 152.465 142.24) (end 155.005 139.7) (width 0.25) (layer "B.Cu") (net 27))
 (segment (start 149.86 142.24) (end 152.465 142.24) (width 0.25) (layer "B.Cu") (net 27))
 (segment (start 175.26 106.68) (end 175.26 107.95) (width 0.25) (layer "F.Cu") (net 44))
 (segment (start 175.26 136.523604) (end 175.26 139.7) (width 0.25) (layer "F.Cu") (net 44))
 (segment (start 173.99 135.253604) (end 175.26 136.523604) (width 0.25) (layer "F.Cu") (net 44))
 (segment (start 175.26 107.95) (end 173.99 109.22) (width 0.25) (layer "F.Cu") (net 44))
 (segment (start 173.99 109.22) (end 173.99 135.253604) (width 0.25) (layer "F.Cu") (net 44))
 (segment (start 149.352 112.268) (end 167.64 112.268) (width 0.25) (layer "B.Cu") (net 44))
 (segment (start 147.32 114.3) (end 149.352 112.268) (width 0.25) (layer "B.Cu") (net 44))
 (segment (start 169.672 112.268) (end 167.64 112.268) (width 0.25) (layer "B.Cu") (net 44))
 (segment (start 175.26 106.68) (end 169.672 112.268) (width 0.25) (layer "B.Cu") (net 44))
 (segment (start 190.5 106.68) (end 190.5 111.76) (width 0.25) (layer "F.Cu") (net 43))
 (segment (start 195.58 106.68) (end 190.5 106.68) (width 0.25) (layer "F.Cu") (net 43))
 (segment (start 175.26 119.38) (end 175.26 123.4795) (width 0.25) (layer "F.Cu") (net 39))
 (via (at 175.26 123.4795) (size 0.8) (drill 0.4) (layers "F.Cu" "B.Cu") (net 39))
 (segment (start 196.755 110.395) (end 196.755 117.255991) (width 0.25) (layer "B.Cu") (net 39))
 (segment (start 196.755 117.255991) (end 190.805991 123.205) (width 0.25) (layer "B.Cu") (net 39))
 (segment (start 190.805991 123.205) (end 175.5345 123.205) (width 0.25) (layer "B.Cu") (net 39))
 (segment (start 195.58 109.22) (end 196.755 110.395) (width 0.25) (layer "B.Cu") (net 39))
 (segment (start 175.5345 123.205) (end 175.26 123.4795) (width 0.25) (layer "B.Cu") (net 39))
 (segment (start 172.72 114.3) (end 172.72 119.38) (width 0.25) (layer "F.Cu") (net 40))
 (segment (start 175.26 116.84) (end 177.8 119.38) (width 0.25) (layer "B.Cu") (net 38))
 (segment (start 175.26 116.84) (end 175.26 114.3) (width 0.25) (layer "B.Cu") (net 38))
 (segment (start 171.305 118.255) (end 171.305 114.124009) (width 0.25) (layer "B.Cu") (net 41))
 (segment (start 176.675 113.175) (end 177.8 114.3) (width 0.25) (layer "B.Cu") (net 41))
 (segment (start 172.254009 113.175) (end 176.675 113.175) (width 0.25) (layer "B.Cu") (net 41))
 (segment (start 171.305 114.124009) (end 172.254009 113.175) (width 0.25) (layer "B.Cu") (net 41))
 (segment (start 170.18 119.38) (end 171.305 118.255) (width 0.25) (layer "B.Cu") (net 41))
 (segment (start 180.34 114.3) (end 178.765 112.725) (width 0.25) (layer "B.Cu") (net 42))
 (segment (start 168.765 118.255) (end 167.64 119.38) (width 0.25) (layer "B.Cu") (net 42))
 (segment (start 178.765 112.725) (end 170.164009 112.725) (width 0.25) (layer "B.Cu") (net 42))
 (segment (start 170.164009 112.725) (end 168.765 114.124009) (width 0.25) (layer "B.Cu") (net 42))
 (segment (start 168.765 114.124009) (end 168.765 118.255) (width 0.25) (layer "B.Cu") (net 42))
 (segment (start 184.15 143.51) (end 184.15 135.89) (width 0.25) (layer "F.Cu") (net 37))
 (segment (start 180.34 147.32) (end 184.15 143.51) (width 0.25) (layer "F.Cu") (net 37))
 (segment (start 184.15 135.89) (end 182.88 134.62) (width 0.25) (layer "F.Cu") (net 37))
 (segment (start 165.1 134.62) (end 165.1 137.16) (width 0.25) (layer "F.Cu") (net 30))
 (segment (start 165.1 137.16) (end 167.64 139.7) (width 0.25) (layer "F.Cu") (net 30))
 (segment (start 170.18 139.7) (end 171.45 140.97) (width 0.25) (layer "B.Cu") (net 48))
 (segment (start 198.12 105.156) (end 197.104 104.14) (width 0.25) (layer "B.Cu") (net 48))
 (segment (start 190.820991 140.97) (end 198.12 133.670991) (width 0.25) (layer "B.Cu") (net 48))
 (segment (start 198.12 133.670991) (end 198.12 105.156) (width 0.25) (layer "B.Cu") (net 48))
 (segment (start 185.42 104.14) (end 182.88 106.68) (width 0.25) (layer "B.Cu") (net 48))
 (segment (start 171.45 140.97) (end 190.820991 140.97) (width 0.25) (layer "B.Cu") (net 48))
 (segment (start 197.104 104.14) (end 185.42 104.14) (width 0.25) (layer "B.Cu") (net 48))
 (segment (start 168.765 143.655) (end 165.1 147.32) (width 0.25) (layer "F.Cu") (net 31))
 (segment (start 168.765 135.745) (end 168.765 143.655) (width 0.25) (layer "F.Cu") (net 31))
 (segment (start 167.64 134.62) (end 168.765 135.745) (width 0.25) (layer "F.Cu") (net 31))
 (segment (start 171.45 135.89) (end 170.18 134.62) (width 0.25) (layer "F.Cu") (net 32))
 (segment (start 167.64 147.32) (end 171.45 143.51) (width 0.25) (layer "F.Cu") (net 32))
 (segment (start 171.45 143.51) (end 171.45 135.89) (width 0.25) (layer "F.Cu") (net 32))
 (segment (start 173.99 135.89) (end 172.72 134.62) (width 0.25) (layer "F.Cu") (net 33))
 (segment (start 170.18 147.32) (end 173.99 143.51) (width 0.25) (layer "F.Cu") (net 33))
 (segment (start 173.99 143.51) (end 173.99 135.89) (width 0.25) (layer "F.Cu") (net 33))
 (segment (start 176.53 143.51) (end 172.72 147.32) (width 0.25) (layer "F.Cu") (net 34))
 (segment (start 175.26 134.62) (end 176.53 135.89) (width 0.25) (layer "F.Cu") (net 34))
 (segment (start 176.53 135.89) (end 176.53 143.51) (width 0.25) (layer "F.Cu") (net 34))
 (segment (start 179.07 143.51) (end 175.26 147.32) (width 0.25) (layer "F.Cu") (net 35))
 (segment (start 177.8 134.62) (end 179.07 135.89) (width 0.25) (layer "F.Cu") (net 35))
 (segment (start 179.07 135.89) (end 179.07 143.51) (width 0.25) (layer "F.Cu") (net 35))
 (segment (start 180.34 134.62) (end 181.61 135.89) (width 0.25) (layer "F.Cu") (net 36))
 (segment (start 181.61 143.51) (end 177.8 147.32) (width 0.25) (layer "F.Cu") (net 36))
 (segment (start 181.61 135.89) (end 181.61 143.51) (width 0.25) (layer "F.Cu") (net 36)))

